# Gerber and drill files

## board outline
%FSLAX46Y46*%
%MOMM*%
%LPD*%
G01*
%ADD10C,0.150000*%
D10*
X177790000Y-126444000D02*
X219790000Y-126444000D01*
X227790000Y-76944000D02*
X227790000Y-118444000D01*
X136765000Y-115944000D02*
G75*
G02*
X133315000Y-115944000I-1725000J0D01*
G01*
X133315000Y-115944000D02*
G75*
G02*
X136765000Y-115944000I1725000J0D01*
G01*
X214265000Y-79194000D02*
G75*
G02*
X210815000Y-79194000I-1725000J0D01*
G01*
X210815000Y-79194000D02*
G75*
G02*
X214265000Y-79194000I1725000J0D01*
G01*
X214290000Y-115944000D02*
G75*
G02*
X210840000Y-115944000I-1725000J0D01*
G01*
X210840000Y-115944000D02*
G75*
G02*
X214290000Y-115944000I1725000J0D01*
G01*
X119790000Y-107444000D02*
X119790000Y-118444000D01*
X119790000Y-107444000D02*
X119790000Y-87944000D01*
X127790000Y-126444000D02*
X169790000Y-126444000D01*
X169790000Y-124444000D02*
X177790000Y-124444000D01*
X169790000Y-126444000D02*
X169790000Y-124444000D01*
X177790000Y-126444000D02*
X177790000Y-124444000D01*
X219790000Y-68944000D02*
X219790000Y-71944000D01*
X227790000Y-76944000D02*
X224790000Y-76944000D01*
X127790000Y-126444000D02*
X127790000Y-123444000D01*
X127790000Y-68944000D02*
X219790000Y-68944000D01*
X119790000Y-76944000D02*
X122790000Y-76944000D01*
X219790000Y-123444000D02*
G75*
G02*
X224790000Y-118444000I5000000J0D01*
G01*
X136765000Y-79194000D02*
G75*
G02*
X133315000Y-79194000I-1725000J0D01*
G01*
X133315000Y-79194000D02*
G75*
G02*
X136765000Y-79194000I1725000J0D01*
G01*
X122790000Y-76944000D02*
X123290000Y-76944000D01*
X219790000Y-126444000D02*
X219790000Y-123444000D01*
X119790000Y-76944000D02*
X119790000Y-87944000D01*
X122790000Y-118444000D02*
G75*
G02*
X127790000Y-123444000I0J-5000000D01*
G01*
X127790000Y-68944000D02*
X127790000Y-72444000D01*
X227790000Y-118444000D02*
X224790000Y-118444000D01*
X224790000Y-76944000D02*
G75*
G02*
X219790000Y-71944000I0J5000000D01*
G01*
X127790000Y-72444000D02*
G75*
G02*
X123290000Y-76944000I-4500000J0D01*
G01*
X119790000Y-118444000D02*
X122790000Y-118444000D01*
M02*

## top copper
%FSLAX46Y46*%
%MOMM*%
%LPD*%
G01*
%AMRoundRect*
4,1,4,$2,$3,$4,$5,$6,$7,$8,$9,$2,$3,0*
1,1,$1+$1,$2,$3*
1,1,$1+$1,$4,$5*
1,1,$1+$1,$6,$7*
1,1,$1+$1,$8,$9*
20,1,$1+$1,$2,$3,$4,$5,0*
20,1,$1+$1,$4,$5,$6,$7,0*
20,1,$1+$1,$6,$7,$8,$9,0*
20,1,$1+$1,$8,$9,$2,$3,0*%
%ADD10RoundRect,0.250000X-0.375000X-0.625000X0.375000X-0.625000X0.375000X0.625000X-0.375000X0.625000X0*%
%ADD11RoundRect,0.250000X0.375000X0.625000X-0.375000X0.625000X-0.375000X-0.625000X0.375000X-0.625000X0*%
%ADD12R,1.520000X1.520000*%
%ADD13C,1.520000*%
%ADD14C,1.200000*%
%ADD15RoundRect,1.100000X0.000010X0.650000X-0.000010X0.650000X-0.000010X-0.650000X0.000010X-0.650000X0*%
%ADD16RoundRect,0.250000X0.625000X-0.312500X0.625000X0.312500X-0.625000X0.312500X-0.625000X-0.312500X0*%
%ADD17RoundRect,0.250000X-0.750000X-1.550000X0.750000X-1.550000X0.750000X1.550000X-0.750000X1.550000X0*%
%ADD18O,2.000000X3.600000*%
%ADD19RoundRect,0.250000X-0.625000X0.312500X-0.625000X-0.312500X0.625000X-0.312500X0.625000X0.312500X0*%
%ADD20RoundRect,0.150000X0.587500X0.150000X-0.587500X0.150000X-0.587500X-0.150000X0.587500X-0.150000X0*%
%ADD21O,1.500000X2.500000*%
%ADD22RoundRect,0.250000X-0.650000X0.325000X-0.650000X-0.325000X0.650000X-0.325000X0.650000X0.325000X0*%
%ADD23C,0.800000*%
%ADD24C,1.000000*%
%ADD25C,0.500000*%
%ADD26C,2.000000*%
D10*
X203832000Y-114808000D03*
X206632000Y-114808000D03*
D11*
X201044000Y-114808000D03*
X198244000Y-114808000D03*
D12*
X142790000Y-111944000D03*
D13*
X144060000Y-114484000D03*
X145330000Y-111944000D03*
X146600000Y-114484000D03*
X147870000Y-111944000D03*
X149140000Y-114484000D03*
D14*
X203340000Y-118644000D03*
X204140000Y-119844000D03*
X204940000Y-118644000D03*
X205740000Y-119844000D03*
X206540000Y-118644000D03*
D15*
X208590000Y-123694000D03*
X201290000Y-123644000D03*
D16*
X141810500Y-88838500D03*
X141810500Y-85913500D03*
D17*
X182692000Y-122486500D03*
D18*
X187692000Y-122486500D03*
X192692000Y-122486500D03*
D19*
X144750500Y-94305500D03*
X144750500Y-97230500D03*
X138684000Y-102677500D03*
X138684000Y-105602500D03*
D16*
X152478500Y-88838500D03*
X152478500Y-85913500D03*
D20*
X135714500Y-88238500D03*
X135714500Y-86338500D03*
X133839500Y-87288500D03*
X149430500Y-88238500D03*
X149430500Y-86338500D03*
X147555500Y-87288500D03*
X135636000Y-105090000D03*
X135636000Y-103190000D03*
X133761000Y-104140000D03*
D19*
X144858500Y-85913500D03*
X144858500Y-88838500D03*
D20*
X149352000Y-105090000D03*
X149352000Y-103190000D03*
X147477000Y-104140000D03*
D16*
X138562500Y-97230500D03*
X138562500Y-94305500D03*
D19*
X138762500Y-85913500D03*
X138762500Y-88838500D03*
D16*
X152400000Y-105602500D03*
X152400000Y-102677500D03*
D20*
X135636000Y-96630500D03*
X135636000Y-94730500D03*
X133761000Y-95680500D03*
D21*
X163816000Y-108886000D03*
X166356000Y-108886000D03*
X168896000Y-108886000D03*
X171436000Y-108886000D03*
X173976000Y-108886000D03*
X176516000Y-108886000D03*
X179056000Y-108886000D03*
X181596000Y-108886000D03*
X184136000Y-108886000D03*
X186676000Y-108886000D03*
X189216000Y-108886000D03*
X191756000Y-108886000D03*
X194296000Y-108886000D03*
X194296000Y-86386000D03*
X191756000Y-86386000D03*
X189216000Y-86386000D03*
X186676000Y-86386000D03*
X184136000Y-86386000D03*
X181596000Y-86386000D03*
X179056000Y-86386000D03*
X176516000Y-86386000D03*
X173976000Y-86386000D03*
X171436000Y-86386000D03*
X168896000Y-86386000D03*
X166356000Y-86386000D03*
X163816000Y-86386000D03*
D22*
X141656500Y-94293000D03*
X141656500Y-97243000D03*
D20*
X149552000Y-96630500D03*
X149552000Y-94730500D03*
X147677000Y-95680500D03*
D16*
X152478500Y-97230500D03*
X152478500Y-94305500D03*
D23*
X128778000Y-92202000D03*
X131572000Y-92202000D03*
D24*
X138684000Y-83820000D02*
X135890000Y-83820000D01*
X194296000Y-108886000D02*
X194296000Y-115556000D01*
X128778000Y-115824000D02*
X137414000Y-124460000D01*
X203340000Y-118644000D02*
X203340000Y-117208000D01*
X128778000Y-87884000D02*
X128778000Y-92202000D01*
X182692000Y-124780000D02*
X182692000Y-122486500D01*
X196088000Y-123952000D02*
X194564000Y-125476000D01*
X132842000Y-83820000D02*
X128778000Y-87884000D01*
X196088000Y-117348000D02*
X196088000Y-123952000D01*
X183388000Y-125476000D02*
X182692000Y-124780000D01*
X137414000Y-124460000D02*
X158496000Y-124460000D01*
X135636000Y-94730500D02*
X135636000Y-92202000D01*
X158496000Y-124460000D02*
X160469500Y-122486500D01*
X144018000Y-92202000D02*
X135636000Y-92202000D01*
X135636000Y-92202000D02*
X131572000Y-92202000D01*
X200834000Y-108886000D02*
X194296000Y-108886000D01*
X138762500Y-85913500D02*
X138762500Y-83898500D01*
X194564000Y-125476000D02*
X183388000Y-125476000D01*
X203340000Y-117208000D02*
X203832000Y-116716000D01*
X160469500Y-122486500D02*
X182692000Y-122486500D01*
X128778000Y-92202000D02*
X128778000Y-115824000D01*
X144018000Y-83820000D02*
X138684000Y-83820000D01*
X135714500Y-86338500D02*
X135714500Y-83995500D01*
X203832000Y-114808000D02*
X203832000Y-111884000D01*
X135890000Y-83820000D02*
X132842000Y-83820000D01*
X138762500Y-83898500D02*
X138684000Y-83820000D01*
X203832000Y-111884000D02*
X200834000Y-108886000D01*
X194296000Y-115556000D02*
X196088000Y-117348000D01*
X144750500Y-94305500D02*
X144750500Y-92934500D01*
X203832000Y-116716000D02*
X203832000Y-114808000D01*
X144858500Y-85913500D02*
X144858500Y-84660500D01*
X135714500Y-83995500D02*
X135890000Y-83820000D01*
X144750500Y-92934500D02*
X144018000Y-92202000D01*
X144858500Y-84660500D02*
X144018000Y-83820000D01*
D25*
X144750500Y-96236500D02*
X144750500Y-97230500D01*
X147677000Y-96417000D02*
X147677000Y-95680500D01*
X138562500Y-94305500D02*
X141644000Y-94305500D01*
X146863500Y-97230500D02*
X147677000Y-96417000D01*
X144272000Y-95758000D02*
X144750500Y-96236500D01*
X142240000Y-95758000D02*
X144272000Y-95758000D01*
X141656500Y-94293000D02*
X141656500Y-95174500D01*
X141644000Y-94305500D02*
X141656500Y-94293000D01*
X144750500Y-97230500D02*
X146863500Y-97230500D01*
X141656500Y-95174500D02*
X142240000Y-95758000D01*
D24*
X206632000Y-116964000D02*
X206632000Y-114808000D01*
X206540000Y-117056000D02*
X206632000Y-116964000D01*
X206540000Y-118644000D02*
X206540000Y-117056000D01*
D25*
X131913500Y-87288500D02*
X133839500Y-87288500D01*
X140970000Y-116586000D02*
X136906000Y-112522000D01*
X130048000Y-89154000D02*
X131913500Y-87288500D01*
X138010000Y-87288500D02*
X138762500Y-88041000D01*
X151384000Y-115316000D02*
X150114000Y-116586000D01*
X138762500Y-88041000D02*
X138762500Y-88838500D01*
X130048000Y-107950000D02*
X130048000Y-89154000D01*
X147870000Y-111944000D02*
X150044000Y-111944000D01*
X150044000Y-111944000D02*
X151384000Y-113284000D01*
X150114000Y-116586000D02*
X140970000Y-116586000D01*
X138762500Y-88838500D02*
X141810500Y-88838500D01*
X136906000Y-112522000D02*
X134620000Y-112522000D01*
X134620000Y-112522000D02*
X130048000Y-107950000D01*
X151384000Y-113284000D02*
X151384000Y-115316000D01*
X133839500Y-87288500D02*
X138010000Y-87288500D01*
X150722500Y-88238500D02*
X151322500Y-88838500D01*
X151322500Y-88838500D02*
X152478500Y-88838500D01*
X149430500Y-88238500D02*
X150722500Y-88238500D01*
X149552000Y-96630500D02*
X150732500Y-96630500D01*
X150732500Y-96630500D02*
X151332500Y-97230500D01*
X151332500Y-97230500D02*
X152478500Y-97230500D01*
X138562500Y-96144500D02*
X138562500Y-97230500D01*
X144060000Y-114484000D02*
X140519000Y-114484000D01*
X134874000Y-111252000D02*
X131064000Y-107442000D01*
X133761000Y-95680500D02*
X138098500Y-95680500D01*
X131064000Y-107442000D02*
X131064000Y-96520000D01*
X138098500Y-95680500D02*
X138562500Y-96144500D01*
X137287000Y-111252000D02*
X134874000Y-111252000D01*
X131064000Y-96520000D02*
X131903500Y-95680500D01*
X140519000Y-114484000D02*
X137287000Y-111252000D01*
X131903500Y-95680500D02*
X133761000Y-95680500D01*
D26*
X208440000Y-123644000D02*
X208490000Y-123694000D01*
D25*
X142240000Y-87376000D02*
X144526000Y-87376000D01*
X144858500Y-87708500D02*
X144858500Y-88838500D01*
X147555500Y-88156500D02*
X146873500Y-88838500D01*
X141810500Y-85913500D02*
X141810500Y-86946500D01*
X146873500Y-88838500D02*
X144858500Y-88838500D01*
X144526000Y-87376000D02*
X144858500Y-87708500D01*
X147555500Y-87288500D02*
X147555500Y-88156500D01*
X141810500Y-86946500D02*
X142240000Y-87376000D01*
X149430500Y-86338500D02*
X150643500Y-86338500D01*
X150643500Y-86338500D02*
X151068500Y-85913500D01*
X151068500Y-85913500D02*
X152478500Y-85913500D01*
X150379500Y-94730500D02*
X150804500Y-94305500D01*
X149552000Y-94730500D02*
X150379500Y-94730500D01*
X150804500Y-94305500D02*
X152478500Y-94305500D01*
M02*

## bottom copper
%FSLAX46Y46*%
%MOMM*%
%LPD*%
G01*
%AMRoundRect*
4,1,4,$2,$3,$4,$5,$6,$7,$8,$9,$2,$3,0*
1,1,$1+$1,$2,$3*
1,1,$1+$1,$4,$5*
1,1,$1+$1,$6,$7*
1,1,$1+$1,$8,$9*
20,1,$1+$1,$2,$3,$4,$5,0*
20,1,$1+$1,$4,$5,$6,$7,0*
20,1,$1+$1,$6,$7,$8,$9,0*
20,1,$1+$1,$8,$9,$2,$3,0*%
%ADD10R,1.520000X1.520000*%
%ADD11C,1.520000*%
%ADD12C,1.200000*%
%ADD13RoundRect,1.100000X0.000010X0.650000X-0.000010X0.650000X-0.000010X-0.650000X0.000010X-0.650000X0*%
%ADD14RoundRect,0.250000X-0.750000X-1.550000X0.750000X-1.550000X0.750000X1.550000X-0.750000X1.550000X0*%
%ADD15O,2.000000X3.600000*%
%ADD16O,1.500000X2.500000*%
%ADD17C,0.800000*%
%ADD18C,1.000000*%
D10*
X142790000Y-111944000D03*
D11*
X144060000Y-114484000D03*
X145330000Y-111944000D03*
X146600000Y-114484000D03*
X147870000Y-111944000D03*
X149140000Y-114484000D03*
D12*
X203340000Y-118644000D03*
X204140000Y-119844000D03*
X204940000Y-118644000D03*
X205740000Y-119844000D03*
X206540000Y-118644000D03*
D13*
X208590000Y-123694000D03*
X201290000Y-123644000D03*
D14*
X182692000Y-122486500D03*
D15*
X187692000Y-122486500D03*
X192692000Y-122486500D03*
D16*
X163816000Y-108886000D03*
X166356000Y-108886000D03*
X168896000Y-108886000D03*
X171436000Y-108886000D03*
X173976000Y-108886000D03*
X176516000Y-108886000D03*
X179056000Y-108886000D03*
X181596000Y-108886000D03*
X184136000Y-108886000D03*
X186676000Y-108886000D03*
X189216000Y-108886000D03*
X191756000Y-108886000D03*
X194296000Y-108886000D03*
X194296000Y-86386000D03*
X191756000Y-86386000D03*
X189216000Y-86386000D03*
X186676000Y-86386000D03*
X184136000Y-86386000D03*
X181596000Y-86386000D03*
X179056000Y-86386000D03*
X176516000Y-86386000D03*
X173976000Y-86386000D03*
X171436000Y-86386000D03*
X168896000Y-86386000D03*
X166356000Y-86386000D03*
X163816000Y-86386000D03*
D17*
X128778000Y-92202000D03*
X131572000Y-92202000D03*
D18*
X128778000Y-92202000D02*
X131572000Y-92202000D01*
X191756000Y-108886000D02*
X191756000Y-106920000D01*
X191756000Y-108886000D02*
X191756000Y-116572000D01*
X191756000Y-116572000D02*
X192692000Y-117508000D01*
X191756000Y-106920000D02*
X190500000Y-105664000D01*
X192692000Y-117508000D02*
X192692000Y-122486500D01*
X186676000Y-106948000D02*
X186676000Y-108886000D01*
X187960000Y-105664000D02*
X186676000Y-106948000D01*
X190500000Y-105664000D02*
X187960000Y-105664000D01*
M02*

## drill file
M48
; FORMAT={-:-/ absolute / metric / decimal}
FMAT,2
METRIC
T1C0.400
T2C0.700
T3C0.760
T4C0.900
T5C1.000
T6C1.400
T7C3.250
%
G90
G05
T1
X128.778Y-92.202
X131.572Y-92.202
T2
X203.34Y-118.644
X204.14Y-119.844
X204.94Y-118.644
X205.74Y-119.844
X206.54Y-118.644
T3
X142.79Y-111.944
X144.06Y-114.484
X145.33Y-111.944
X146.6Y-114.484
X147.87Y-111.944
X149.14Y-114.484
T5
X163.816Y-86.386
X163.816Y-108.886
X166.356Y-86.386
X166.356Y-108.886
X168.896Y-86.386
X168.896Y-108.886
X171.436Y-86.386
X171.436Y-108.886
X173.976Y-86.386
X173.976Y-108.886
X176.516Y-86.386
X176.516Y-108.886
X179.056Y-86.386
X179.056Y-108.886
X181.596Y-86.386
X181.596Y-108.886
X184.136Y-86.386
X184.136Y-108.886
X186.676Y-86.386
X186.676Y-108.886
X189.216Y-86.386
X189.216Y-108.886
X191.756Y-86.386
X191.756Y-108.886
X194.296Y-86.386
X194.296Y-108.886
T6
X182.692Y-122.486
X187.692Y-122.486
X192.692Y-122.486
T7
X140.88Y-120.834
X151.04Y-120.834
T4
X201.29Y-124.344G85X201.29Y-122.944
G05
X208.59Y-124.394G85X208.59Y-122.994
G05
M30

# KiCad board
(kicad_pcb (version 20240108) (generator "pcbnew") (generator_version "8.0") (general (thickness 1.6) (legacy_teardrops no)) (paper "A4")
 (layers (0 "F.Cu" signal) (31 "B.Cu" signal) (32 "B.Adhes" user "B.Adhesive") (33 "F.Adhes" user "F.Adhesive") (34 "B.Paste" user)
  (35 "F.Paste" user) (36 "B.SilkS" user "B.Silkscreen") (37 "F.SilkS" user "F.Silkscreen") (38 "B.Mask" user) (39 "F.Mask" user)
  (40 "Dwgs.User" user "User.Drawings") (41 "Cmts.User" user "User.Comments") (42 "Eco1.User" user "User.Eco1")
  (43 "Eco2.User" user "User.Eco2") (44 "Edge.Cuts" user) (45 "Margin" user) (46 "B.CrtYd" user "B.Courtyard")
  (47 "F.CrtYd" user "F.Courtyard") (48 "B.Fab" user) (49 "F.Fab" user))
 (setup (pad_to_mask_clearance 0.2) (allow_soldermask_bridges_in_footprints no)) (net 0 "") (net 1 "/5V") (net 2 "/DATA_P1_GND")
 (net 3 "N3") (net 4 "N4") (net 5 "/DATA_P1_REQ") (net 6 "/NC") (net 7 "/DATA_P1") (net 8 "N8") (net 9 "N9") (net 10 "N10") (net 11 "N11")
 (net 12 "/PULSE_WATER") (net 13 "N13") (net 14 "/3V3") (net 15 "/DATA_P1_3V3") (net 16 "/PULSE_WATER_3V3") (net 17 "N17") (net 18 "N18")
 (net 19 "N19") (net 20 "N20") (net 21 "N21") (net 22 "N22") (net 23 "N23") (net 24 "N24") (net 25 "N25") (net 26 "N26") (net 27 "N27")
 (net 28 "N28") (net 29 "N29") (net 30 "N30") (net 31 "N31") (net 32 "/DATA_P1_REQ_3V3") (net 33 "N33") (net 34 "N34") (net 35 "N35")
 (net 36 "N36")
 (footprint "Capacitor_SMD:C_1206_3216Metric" (layer "F.Cu") (at 205.232 114.808)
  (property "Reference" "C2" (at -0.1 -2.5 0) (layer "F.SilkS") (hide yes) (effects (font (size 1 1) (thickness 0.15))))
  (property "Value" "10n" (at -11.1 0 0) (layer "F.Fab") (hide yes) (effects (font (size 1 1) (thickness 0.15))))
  (pad "1" smd roundrect (at -1.4 0) (size 1.25 1.75) (layers "F.Cu" "F.Paste" "F.Mask") (roundrect_rratio 0.2) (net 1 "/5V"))
  (pad "2" smd roundrect (at 1.4 0) (size 1.25 1.75) (layers "F.Cu" "F.Paste" "F.Mask") (roundrect_rratio 0.2) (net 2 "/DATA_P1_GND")))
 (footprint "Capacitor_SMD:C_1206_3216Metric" (layer "F.Cu") (at 199.644 114.808 180)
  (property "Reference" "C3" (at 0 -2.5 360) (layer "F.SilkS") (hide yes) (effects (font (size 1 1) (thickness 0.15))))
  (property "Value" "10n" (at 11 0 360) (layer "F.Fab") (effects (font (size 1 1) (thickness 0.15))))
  (pad "1" smd roundrect (at -1.4 0 180) (size 1.25 1.75) (layers "F.Cu" "F.Paste" "F.Mask") (roundrect_rratio 0.2) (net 2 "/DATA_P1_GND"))
  (pad "2" smd roundrect (at 1.4 0 180) (size 1.25 1.75) (layers "F.Cu" "F.Paste" "F.Mask") (roundrect_rratio 0.2) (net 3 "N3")))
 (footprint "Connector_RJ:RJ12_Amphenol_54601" (layer "F.Cu") (at 142.79 111.944)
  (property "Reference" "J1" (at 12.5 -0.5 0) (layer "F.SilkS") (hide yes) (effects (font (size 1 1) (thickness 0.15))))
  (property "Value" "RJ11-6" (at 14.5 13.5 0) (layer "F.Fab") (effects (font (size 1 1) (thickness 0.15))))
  (pad "" np_thru_hole circle (at -1.91 8.89) (size 3.25 3.25) (drill 3.25) (layers "*.Cu" "*.Mask"))
  (pad "" np_thru_hole circle (at 8.25 8.89) (size 3.25 3.25) (drill 3.25) (layers "*.Cu" "*.Mask"))
  (pad "1" thru_hole rect (at 0 0) (size 1.52 1.52) (drill 0.76) (layers "*.Cu" "*.Mask") (remove_unused_layers no) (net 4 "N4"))
  (pad "2" thru_hole circle (at 1.27 2.54) (size 1.52 1.52) (drill 0.76) (layers "*.Cu" "*.Mask") (remove_unused_layers no)
   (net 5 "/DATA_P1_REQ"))
  (pad "3" thru_hole circle (at 2.54 0) (size 1.52 1.52) (drill 0.76) (layers "*.Cu" "*.Mask") (remove_unused_layers no)
   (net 2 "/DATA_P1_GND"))
  (pad "4" thru_hole circle (at 3.81 2.54) (size 1.52 1.52) (drill 0.76) (layers "*.Cu" "*.Mask") (remove_unused_layers no) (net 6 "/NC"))
  (pad "5" thru_hole circle (at 5.08 0) (size 1.52 1.52) (drill 0.76) (layers "*.Cu" "*.Mask") (remove_unused_layers no) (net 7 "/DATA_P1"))
  (pad "6" thru_hole circle (at 6.35 2.54) (size 1.52 1.52) (drill 0.76) (layers "*.Cu" "*.Mask") (remove_unused_layers no)
   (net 2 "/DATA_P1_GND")))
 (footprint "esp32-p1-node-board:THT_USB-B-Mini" (layer "F.Cu") (at 208.79 127.444 90)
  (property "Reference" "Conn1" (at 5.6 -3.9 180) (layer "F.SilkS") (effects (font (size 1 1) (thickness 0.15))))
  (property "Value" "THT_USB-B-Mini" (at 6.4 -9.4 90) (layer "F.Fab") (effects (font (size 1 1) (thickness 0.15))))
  (pad "1" thru_hole circle (at 8.8 -5.45 180) (size 1.2 1.2) (drill 0.7) (layers "*.Cu" "*.Mask") (remove_unused_layers no) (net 1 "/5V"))
  (pad "2" thru_hole circle (at 7.6 -4.65 180) (size 1.2 1.2) (drill 0.7) (layers "*.Cu" "*.Mask") (remove_unused_layers no) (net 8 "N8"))
  (pad "3" thru_hole circle (at 8.8 -3.85 180) (size 1.2 1.2) (drill 0.7) (layers "*.Cu" "*.Mask") (remove_unused_layers no) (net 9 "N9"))
  (pad "4" thru_hole circle (at 7.6 -3.05 180) (size 1.2 1.2) (drill 0.7) (layers "*.Cu" "*.Mask") (remove_unused_layers no) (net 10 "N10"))
  (pad "5" thru_hole circle (at 8.8 -2.25 180) (size 1.2 1.2) (drill 0.7) (layers "*.Cu" "*.Mask") (remove_unused_layers no)
   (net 2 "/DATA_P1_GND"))
  (pad "6" thru_hole roundrect (at 3.75 -0.2 180) (size 2.2 3.5) (drill oval 0.9 2.3) (layers "*.Cu" "*.Mask") (remove_unused_layers no)
   (roundrect_rratio 0.5) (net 3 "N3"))
  (pad "7" thru_hole roundrect (at 3.8 -7.5 180) (size 2.2 3.5) (drill oval 0.9 2.3) (layers "*.Cu" "*.Mask") (remove_unused_layers no)
   (roundrect_rratio 0.5) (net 3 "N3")))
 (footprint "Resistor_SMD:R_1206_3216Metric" (layer "F.Cu") (at 141.8105 87.376 90)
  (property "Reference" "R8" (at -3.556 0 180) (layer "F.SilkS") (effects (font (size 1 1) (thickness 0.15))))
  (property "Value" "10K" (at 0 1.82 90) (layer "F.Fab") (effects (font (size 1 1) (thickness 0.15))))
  (pad "1" smd roundrect (at -1.4625 0 90) (size 1.125 1.75) (layers "F.Cu" "F.Paste" "F.Mask") (roundrect_rratio 0.222222)
   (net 7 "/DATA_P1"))
  (pad "2" smd roundrect (at 1.4625 0 90) (size 1.125 1.75) (layers "F.Cu" "F.Paste" "F.Mask") (roundrect_rratio 0.222222) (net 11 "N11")))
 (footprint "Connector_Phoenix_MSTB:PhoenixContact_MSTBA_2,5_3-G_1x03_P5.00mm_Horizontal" (layer "F.Cu") (at 182.692 122.4865)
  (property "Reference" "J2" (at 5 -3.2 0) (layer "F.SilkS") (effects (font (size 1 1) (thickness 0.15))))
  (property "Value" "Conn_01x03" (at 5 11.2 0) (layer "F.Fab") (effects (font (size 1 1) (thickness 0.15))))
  (pad "1" thru_hole roundrect (at 0 0) (size 2 3.6) (drill 1.4) (layers "*.Cu" "*.Mask") (remove_unused_layers no) (roundrect_rratio 0.125)
   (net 1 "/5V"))
  (pad "2" thru_hole oval (at 5 0) (size 2 3.6) (drill 1.4) (layers "*.Cu" "*.Mask") (remove_unused_layers no) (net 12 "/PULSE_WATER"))
  (pad "3" thru_hole oval (at 10 0) (size 2 3.6) (drill 1.4) (layers "*.Cu" "*.Mask") (remove_unused_layers no) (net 2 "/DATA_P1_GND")))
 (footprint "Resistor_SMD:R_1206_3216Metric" (layer "F.Cu") (at 144.7505 95.768 -90)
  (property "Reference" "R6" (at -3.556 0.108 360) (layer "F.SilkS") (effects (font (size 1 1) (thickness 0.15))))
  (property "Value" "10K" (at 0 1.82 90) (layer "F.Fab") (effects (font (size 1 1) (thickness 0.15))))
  (pad "1" smd roundrect (at -1.4625 0 270) (size 1.125 1.75) (layers "F.Cu" "F.Paste" "F.Mask") (roundrect_rratio 0.222222) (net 1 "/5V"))
  (pad "2" smd roundrect (at 1.4625 0 270) (size 1.125 1.75) (layers "F.Cu" "F.Paste" "F.Mask") (roundrect_rratio 0.222222) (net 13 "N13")))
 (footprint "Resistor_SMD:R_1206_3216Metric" (layer "F.Cu") (at 138.684 104.14 -90)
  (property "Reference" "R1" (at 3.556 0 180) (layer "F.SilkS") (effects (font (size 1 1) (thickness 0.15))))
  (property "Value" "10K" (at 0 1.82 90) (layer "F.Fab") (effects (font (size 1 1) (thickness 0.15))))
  (pad "1" smd roundrect (at -1.4625 0 270) (size 1.125 1.75) (layers "F.Cu" "F.Paste" "F.Mask") (roundrect_rratio 0.222222) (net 1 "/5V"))
  (pad "2" smd roundrect (at 1.4625 0 270) (size 1.125 1.75) (layers "F.Cu" "F.Paste" "F.Mask") (roundrect_rratio 0.222222)
   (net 12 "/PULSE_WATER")))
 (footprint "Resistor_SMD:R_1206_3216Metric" (layer "F.Cu") (at 152.4785 87.376 90)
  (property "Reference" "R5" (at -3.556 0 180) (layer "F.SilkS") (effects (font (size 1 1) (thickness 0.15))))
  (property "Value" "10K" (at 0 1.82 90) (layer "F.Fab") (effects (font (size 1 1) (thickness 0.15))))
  (pad "1" smd roundrect (at -1.4625 0 90) (size 1.125 1.75) (layers "F.Cu" "F.Paste" "F.Mask") (roundrect_rratio 0.222222) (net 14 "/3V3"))
  (pad "2" smd roundrect (at 1.4625 0 90) (size 1.125 1.75) (layers "F.Cu" "F.Paste" "F.Mask") (roundrect_rratio 0.222222)
   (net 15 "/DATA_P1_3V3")))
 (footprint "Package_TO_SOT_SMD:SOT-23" (layer "F.Cu") (at 134.777 87.2885 180)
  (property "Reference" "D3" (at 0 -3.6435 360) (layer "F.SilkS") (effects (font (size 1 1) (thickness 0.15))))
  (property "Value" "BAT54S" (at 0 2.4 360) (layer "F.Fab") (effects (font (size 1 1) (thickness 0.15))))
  (pad "1" smd roundrect (at -0.9375 -0.95 180) (size 1.475 0.6) (layers "F.Cu" "F.Paste" "F.Mask") (roundrect_rratio 0.25)
   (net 2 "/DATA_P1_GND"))
  (pad "2" smd roundrect (at -0.9375 0.95 180) (size 1.475 0.6) (layers "F.Cu" "F.Paste" "F.Mask") (roundrect_rratio 0.25) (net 1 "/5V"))
  (pad "3" smd roundrect (at 0.9375 0 180) (size 1.475 0.6) (layers "F.Cu" "F.Paste" "F.Mask") (roundrect_rratio 0.25) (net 7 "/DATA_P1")))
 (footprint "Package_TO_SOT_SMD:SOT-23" (layer "F.Cu") (at 148.493 87.2885 180)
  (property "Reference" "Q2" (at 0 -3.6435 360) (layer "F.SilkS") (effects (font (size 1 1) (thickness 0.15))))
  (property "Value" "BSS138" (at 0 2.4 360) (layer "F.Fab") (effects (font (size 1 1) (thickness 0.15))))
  (pad "1" smd roundrect (at -0.9375 -0.95 180) (size 1.475 0.6) (layers "F.Cu" "F.Paste" "F.Mask") (roundrect_rratio 0.25) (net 14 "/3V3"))
  (pad "2" smd roundrect (at -0.9375 0.95 180) (size 1.475 0.6) (layers "F.Cu" "F.Paste" "F.Mask") (roundrect_rratio 0.25)
   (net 15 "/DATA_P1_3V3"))
  (pad "3" smd roundrect (at 0.9375 0 180) (size 1.475 0.6) (layers "F.Cu" "F.Paste" "F.Mask") (roundrect_rratio 0.25) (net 11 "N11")))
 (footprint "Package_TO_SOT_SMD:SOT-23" (layer "F.Cu") (at 134.6985 104.14 180)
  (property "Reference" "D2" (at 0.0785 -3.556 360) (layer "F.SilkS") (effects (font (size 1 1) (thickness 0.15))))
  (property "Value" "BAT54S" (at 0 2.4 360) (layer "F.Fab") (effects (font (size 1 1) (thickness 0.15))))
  (pad "1" smd roundrect (at -0.9375 -0.95 180) (size 1.475 0.6) (layers "F.Cu" "F.Paste" "F.Mask") (roundrect_rratio 0.25)
   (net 2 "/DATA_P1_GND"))
  (pad "2" smd roundrect (at -0.9375 0.95 180) (size 1.475 0.6) (layers "F.Cu" "F.Paste" "F.Mask") (roundrect_rratio 0.25) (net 1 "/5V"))
  (pad "3" smd roundrect (at 0.9375 0 180) (size 1.475 0.6) (layers "F.Cu" "F.Paste" "F.Mask") (roundrect_rratio 0.25)
   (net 12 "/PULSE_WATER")))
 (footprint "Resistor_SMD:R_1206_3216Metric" (layer "F.Cu") (at 144.8585 87.376 -90)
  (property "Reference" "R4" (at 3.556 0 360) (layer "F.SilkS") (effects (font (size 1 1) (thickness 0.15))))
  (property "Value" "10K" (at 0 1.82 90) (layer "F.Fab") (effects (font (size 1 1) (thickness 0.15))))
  (pad "1" smd roundrect (at -1.4625 0 270) (size 1.125 1.75) (layers "F.Cu" "F.Paste" "F.Mask") (roundrect_rratio 0.222222) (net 1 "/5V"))
  (pad "2" smd roundrect (at 1.4625 0 270) (size 1.125 1.75) (layers "F.Cu" "F.Paste" "F.Mask") (roundrect_rratio 0.222222) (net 11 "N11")))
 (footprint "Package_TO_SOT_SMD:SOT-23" (layer "F.Cu") (at 148.4145 104.14 180)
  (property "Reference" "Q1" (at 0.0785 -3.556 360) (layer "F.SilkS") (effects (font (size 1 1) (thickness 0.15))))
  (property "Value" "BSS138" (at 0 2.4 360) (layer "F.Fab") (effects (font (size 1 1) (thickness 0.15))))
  (pad "1" smd roundrect (at -0.9375 -0.95 180) (size 1.475 0.6) (layers "F.Cu" "F.Paste" "F.Mask") (roundrect_rratio 0.25) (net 14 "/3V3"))
  (pad "2" smd roundrect (at -0.9375 0.95 180) (size 1.475 0.6) (layers "F.Cu" "F.Paste" "F.Mask") (roundrect_rratio 0.25)
   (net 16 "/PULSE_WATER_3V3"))
  (pad "3" smd roundrect (at 0.9375 0 180) (size 1.475 0.6) (layers "F.Cu" "F.Paste" "F.Mask") (roundrect_rratio 0.25)
   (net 12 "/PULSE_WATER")))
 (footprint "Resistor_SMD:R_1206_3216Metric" (layer "F.Cu") (at 138.5625 95.768 90)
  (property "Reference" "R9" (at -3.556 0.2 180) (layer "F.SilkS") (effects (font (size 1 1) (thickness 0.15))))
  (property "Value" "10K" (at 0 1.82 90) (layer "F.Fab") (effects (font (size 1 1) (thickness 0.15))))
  (pad "1" smd roundrect (at -1.4625 0 90) (size 1.125 1.75) (layers "F.Cu" "F.Paste" "F.Mask") (roundrect_rratio 0.222222)
   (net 5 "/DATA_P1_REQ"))
  (pad "2" smd roundrect (at 1.4625 0 90) (size 1.125 1.75) (layers "F.Cu" "F.Paste" "F.Mask") (roundrect_rratio 0.222222) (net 13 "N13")))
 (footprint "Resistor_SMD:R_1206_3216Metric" (layer "F.Cu") (at 138.7625 87.376 -90)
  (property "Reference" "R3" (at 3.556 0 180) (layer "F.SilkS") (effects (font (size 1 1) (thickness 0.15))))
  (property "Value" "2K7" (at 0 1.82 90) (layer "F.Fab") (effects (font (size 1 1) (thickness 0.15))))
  (pad "1" smd roundrect (at -1.4625 0 270) (size 1.125 1.75) (layers "F.Cu" "F.Paste" "F.Mask") (roundrect_rratio 0.222222) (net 1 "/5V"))
  (pad "2" smd roundrect (at 1.4625 0 270) (size 1.125 1.75) (layers "F.Cu" "F.Paste" "F.Mask") (roundrect_rratio 0.222222)
   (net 7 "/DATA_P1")))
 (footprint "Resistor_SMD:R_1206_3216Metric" (layer "F.Cu") (at 152.4 104.14 90)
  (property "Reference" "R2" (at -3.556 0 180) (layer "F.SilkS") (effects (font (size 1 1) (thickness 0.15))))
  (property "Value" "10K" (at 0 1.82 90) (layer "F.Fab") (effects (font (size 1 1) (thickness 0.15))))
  (pad "1" smd roundrect (at -1.4625 0 90) (size 1.125 1.75) (layers "F.Cu" "F.Paste" "F.Mask") (roundrect_rratio 0.222222) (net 14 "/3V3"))
  (pad "2" smd roundrect (at 1.4625 0 90) (size 1.125 1.75) (layers "F.Cu" "F.Paste" "F.Mask") (roundrect_rratio 0.222222)
   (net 16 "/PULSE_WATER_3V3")))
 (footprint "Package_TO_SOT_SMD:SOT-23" (layer "F.Cu") (at 134.6985 95.6805 180)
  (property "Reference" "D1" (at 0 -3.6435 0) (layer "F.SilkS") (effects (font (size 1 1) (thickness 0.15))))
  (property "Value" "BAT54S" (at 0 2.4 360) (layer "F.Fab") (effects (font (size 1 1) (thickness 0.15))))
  (pad "1" smd roundrect (at -0.9375 -0.95 180) (size 1.475 0.6) (layers "F.Cu" "F.Paste" "F.Mask") (roundrect_rratio 0.25)
   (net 2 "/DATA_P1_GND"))
  (pad "2" smd roundrect (at -0.9375 0.95 180) (size 1.475 0.6) (layers "F.Cu" "F.Paste" "F.Mask") (roundrect_rratio 0.25) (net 1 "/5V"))
  (pad "3" smd roundrect (at 0.9375 0 180) (size 1.475 0.6) (layers "F.Cu" "F.Paste" "F.Mask") (roundrect_rratio 0.25)
   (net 5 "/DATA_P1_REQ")))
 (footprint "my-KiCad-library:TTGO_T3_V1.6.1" (layer "F.Cu") (at 179.056 97.636)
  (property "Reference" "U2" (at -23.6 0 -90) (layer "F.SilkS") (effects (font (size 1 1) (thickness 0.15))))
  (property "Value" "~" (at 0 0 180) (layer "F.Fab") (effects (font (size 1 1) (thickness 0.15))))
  (pad "1" thru_hole oval (at -15.24 11.25) (size 1.5 2.5) (drill 1) (layers "*.Cu" "*.Mask") (remove_unused_layers no) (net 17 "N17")
   (thermal_bridge_angle 45))
  (pad "2" thru_hole oval (at -12.7 11.25) (size 1.5 2.5) (drill 1) (layers "*.Cu" "*.Mask") (remove_unused_layers no) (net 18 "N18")
   (thermal_bridge_angle 45))
  (pad "3" thru_hole oval (at -10.16 11.25) (size 1.5 2.5) (drill 1) (layers "*.Cu" "*.Mask") (remove_unused_layers no) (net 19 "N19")
   (thermal_bridge_angle 45))
  (pad "4" thru_hole oval (at -7.62 11.25) (size 1.5 2.5) (drill 1) (layers "*.Cu" "*.Mask") (remove_unused_layers no) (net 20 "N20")
   (thermal_bridge_angle 45))
  (pad "5" thru_hole oval (at -5.08 11.25) (size 1.5 2.5) (drill 1) (layers "*.Cu" "*.Mask") (remove_unused_layers no) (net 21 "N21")
   (thermal_bridge_angle 45))
  (pad "6" thru_hole oval (at -2.54 11.25) (size 1.5 2.5) (drill 1) (layers "*.Cu" "*.Mask") (remove_unused_layers no) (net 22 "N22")
   (thermal_bridge_angle 45))
  (pad "7" thru_hole oval (at 0 11.25) (size 1.5 2.5) (drill 1) (layers "*.Cu" "*.Mask") (remove_unused_layers no) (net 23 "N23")
   (thermal_bridge_angle 45))
  (pad "8" thru_hole oval (at 2.54 11.25) (size 1.5 2.5) (drill 1) (layers "*.Cu" "*.Mask") (remove_unused_layers no) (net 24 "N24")
   (thermal_bridge_angle 45))
  (pad "9" thru_hole oval (at 5.08 11.25) (size 1.5 2.5) (drill 1) (layers "*.Cu" "*.Mask") (remove_unused_layers no) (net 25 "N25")
   (thermal_bridge_angle 45))
  (pad "10" thru_hole oval (at 7.62 11.25) (size 1.5 2.5) (drill 1) (layers "*.Cu" "*.Mask") (remove_unused_layers no)
   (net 2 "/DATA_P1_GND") (thermal_bridge_angle 45))
  (pad "11" thru_hole oval (at 10.16 11.25) (size 1.5 2.5) (drill 1) (layers "*.Cu" "*.Mask") (remove_unused_layers no) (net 14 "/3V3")
   (thermal_bridge_angle 45))
  (pad "12" thru_hole oval (at 12.7 11.25) (size 1.5 2.5) (drill 1) (layers "*.Cu" "*.Mask") (remove_unused_layers no)
   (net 2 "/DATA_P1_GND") (thermal_bridge_angle 45))
  (pad "13" thru_hole oval (at 15.24 11.25) (size 1.5 2.5) (drill 1) (layers "*.Cu" "*.Mask") (remove_unused_layers no) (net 1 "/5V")
   (thermal_bridge_angle 45))
  (pad "14" thru_hole oval (at 15.24 -11.25) (size 1.5 2.5) (drill 1) (layers "*.Cu" "*.Mask") (remove_unused_layers no) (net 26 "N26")
   (thermal_bridge_angle 45))
  (pad "15" thru_hole oval (at 12.7 -11.25) (size 1.5 2.5) (drill 1) (layers "*.Cu" "*.Mask") (remove_unused_layers no)
   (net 16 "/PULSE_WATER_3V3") (thermal_bridge_angle 45))
  (pad "16" thru_hole oval (at 10.16 -11.25) (size 1.5 2.5) (drill 1) (layers "*.Cu" "*.Mask") (remove_unused_layers no) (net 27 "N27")
   (thermal_bridge_angle 45))
  (pad "17" thru_hole oval (at 7.62 -11.25) (size 1.5 2.5) (drill 1) (layers "*.Cu" "*.Mask") (remove_unused_layers no) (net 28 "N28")
   (thermal_bridge_angle 45))
  (pad "18" thru_hole oval (at 5.08 -11.25) (size 1.5 2.5) (drill 1) (layers "*.Cu" "*.Mask") (remove_unused_layers no) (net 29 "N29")
   (thermal_bridge_angle 45))
  (pad "19" thru_hole oval (at 2.54 -11.25) (size 1.5 2.5) (drill 1) (layers "*.Cu" "*.Mask") (remove_unused_layers no) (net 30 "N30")
   (thermal_bridge_angle 45))
  (pad "20" thru_hole oval (at 0 -11.25) (size 1.5 2.5) (drill 1) (layers "*.Cu" "*.Mask") (remove_unused_layers no) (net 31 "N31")
   (thermal_bridge_angle 45))
  (pad "21" thru_hole oval (at -2.54 -11.25) (size 1.5 2.5) (drill 1) (layers "*.Cu" "*.Mask") (remove_unused_layers no)
   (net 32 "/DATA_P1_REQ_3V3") (thermal_bridge_angle 45))
  (pad "22" thru_hole oval (at -5.08 -11.25) (size 1.5 2.5) (drill 1) (layers "*.Cu" "*.Mask") (remove_unused_layers no) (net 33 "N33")
   (thermal_bridge_angle 45))
  (pad "23" thru_hole oval (at -7.62 -11.25) (size 1.5 2.5) (drill 1) (layers "*.Cu" "*.Mask") (remove_unused_layers no)
   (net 15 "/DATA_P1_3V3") (thermal_bridge_angle 45))
  (pad "24" thru_hole oval (at -10.16 -11.25) (size 1.5 2.5) (drill 1) (layers "*.Cu" "*.Mask") (remove_unused_layers no) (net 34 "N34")
   (thermal_bridge_angle 45))
  (pad "25" thru_hole oval (at -12.7 -11.25) (size 1.5 2.5) (drill 1) (layers "*.Cu" "*.Mask") (remove_unused_layers no) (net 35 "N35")
   (thermal_bridge_angle 45))
  (pad "26" thru_hole oval (at -15.24 -11.25) (size 1.5 2.5) (drill 1) (layers "*.Cu" "*.Mask") (remove_unused_layers no) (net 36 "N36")
   (thermal_bridge_angle 45)))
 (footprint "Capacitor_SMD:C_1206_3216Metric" (layer "F.Cu") (at 141.6565 95.768 -90)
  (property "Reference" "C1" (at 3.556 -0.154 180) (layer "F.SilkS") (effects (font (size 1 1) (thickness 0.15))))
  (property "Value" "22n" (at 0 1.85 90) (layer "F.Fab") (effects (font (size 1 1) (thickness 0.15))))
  (pad "1" smd roundrect (at -1.475 0 270) (size 1.15 1.8) (layers "F.Cu" "F.Paste" "F.Mask") (roundrect_rratio 0.217391) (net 13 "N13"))
  (pad "2" smd roundrect (at 1.475 0 270) (size 1.15 1.8) (layers "F.Cu" "F.Paste" "F.Mask") (roundrect_rratio 0.217391)
   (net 2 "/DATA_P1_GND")))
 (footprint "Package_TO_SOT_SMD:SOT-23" (layer "F.Cu") (at 148.6145 95.6805 180)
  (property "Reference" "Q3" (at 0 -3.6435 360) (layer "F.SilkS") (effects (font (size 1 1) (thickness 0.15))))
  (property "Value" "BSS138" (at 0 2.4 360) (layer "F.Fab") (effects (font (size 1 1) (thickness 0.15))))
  (pad "1" smd roundrect (at -0.9375 -0.95 180) (size 1.475 0.6) (layers "F.Cu" "F.Paste" "F.Mask") (roundrect_rratio 0.25) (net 14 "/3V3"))
  (pad "2" smd roundrect (at -0.9375 0.95 180) (size 1.475 0.6) (layers "F.Cu" "F.Paste" "F.Mask") (roundrect_rratio 0.25)
   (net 32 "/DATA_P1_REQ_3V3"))
  (pad "3" smd roundrect (at 0.9375 0 180) (size 1.475 0.6) (layers "F.Cu" "F.Paste" "F.Mask") (roundrect_rratio 0.25) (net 13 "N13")))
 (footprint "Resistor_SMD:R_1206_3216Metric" (layer "F.Cu") (at 152.4785 95.768 90)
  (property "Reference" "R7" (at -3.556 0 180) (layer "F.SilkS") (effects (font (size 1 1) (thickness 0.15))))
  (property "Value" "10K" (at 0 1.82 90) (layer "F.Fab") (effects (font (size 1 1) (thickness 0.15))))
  (pad "1" smd roundrect (at -1.4625 0 90) (size 1.125 1.75) (layers "F.Cu" "F.Paste" "F.Mask") (roundrect_rratio 0.222222) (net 14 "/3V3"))
  (pad "2" smd roundrect (at 1.4625 0 90) (size 1.125 1.75) (layers "F.Cu" "F.Paste" "F.Mask") (roundrect_rratio 0.222222)
   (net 32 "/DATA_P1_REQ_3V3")))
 (gr_line (start 177.79 126.444) (end 219.79 126.444) (stroke (width 0.15) (type solid)) (layer "Edge.Cuts"))
 (gr_line (start 227.79 76.944) (end 227.79 118.444) (stroke (width 0.15) (type solid)) (layer "Edge.Cuts"))
 (gr_circle (center 135.04 115.944) (end 136.765 115.944) (stroke (width 0.15) (type solid)) (fill none) (layer "Edge.Cuts"))
 (gr_circle (center 212.54 79.194) (end 214.265 79.194) (stroke (width 0.15) (type solid)) (fill none) (layer "Edge.Cuts"))
 (gr_circle (center 212.565 115.944) (end 214.29 115.944) (stroke (width 0.15) (type solid)) (fill none) (layer "Edge.Cuts"))
 (gr_line (start 119.79 107.444) (end 119.79 118.444) (stroke (width 0.15) (type solid)) (layer "Edge.Cuts"))
 (gr_line (start 119.79 107.444) (end 119.79 87.944) (stroke (width 0.15) (type solid)) (layer "Edge.Cuts"))
 (gr_line (start 127.79 126.444) (end 169.79 126.444) (stroke (width 0.15) (type solid)) (layer "Edge.Cuts"))
 (gr_line (start 169.79 124.444) (end 177.79 124.444) (stroke (width 0.15) (type solid)) (layer "Edge.Cuts"))
 (gr_line (start 169.79 126.444) (end 169.79 124.444) (stroke (width 0.15) (type solid)) (layer "Edge.Cuts"))
 (gr_line (start 177.79 126.444) (end 177.79 124.444) (stroke (width 0.15) (type solid)) (layer "Edge.Cuts"))
 (gr_line (start 219.79 68.944) (end 219.79 71.944) (stroke (width 0.15) (type solid)) (layer "Edge.Cuts"))
 (gr_line (start 227.79 76.944) (end 224.79 76.944) (stroke (width 0.15) (type solid)) (layer "Edge.Cuts"))
 (gr_line (start 127.79 126.444) (end 127.79 123.444) (stroke (width 0.15) (type solid)) (layer "Edge.Cuts"))
 (gr_line (start 127.79 68.944) (end 219.79 68.944) (stroke (width 0.15) (type solid)) (layer "Edge.Cuts"))
 (gr_line (start 119.79 76.944) (end 122.79 76.944) (stroke (width 0.15) (type solid)) (layer "Edge.Cuts"))
 (gr_arc (start 219.79 123.444) (mid 221.254466 119.908466) (end 224.79 118.444) (stroke (width 0.15) (type solid)) (layer "Edge.Cuts"))
 (gr_circle (center 135.04 79.194) (end 136.765 79.194) (stroke (width 0.15) (type solid)) (fill none) (layer "Edge.Cuts"))
 (gr_line (start 122.79 76.944) (end 123.29 76.944) (stroke (width 0.15) (type solid)) (layer "Edge.Cuts"))
 (gr_line (start 219.79 126.444) (end 219.79 123.444) (stroke (width 0.15) (type solid)) (layer "Edge.Cuts"))
 (gr_line (start 119.79 76.944) (end 119.79 87.944) (stroke (width 0.15) (type solid)) (layer "Edge.Cuts"))
 (gr_arc (start 122.79 118.444) (mid 126.325534 119.908466) (end 127.79 123.444) (stroke (width 0.15) (type solid)) (layer "Edge.Cuts"))
 (gr_line (start 127.79 68.944) (end 127.79 72.444) (stroke (width 0.15) (type solid)) (layer "Edge.Cuts"))
 (gr_line (start 227.79 118.444) (end 224.79 118.444) (stroke (width 0.15) (type solid)) (layer "Edge.Cuts"))
 (gr_arc (start 224.79 76.944) (mid 221.254466 75.479534) (end 219.79 71.944) (stroke (width 0.15) (type solid)) (layer "Edge.Cuts"))
 (gr_arc (start 127.79 72.444) (mid 126.471981 75.625981) (end 123.29 76.944) (stroke (width 0.15) (type solid)) (layer "Edge.Cuts"))
 (gr_line (start 119.79 118.444) (end 122.79 118.444) (stroke (width 0.15) (type solid)) (layer "Edge.Cuts"))
 (segment (start 138.684 83.82) (end 135.89 83.82) (width 1) (layer "F.Cu") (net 1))
 (segment (start 194.296 108.886) (end 194.296 115.556) (width 1) (layer "F.Cu") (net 1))
 (segment (start 128.778 115.824) (end 137.414 124.46) (width 1) (layer "F.Cu") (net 1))
 (segment (start 203.34 118.644) (end 203.34 117.208) (width 1) (layer "F.Cu") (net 1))
 (segment (start 128.778 87.884) (end 128.778 92.202) (width 1) (layer "F.Cu") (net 1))
 (segment (start 182.692 124.78) (end 182.692 122.4865) (width 1) (layer "F.Cu") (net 1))
 (segment (start 196.088 123.952) (end 194.564 125.476) (width 1) (layer "F.Cu") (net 1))
 (segment (start 132.842 83.82) (end 128.778 87.884) (width 1) (layer "F.Cu") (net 1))
 (segment (start 196.088 117.348) (end 196.088 123.952) (width 1) (layer "F.Cu") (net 1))
 (segment (start 183.388 125.476) (end 182.692 124.78) (width 1) (layer "F.Cu") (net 1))
 (segment (start 137.414 124.46) (end 158.496 124.46) (width 1) (layer "F.Cu") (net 1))
 (segment (start 135.636 94.7305) (end 135.636 92.202) (width 1) (layer "F.Cu") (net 1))
 (segment (start 158.496 124.46) (end 160.4695 122.4865) (width 1) (layer "F.Cu") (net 1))
 (segment (start 144.018 92.202) (end 135.636 92.202) (width 1) (layer "F.Cu") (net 1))
 (segment (start 135.636 92.202) (end 131.572 92.202) (width 1) (layer "F.Cu") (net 1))
 (segment (start 200.834 108.886) (end 194.296 108.886) (width 1) (layer "F.Cu") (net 1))
 (segment (start 138.7625 85.9135) (end 138.7625 83.8985) (width 1) (layer "F.Cu") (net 1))
 (segment (start 194.564 125.476) (end 183.388 125.476) (width 1) (layer "F.Cu") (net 1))
 (segment (start 203.34 117.208) (end 203.832 116.716) (width 1) (layer "F.Cu") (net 1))
 (segment (start 160.4695 122.4865) (end 182.692 122.4865) (width 1) (layer "F.Cu") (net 1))
 (segment (start 128.778 92.202) (end 128.778 115.824) (width 1) (layer "F.Cu") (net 1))
 (segment (start 144.018 83.82) (end 138.684 83.82) (width 1) (layer "F.Cu") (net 1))
 (segment (start 135.7145 86.3385) (end 135.7145 83.9955) (width 1) (layer "F.Cu") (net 1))
 (segment (start 203.832 114.808) (end 203.832 111.884) (width 1) (layer "F.Cu") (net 1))
 (segment (start 135.89 83.82) (end 132.842 83.82) (width 1) (layer "F.Cu") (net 1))
 (segment (start 138.7625 83.8985) (end 138.684 83.82) (width 1) (layer "F.Cu") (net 1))
 (segment (start 203.832 111.884) (end 200.834 108.886) (width 1) (layer "F.Cu") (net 1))
 (segment (start 194.296 115.556) (end 196.088 117.348) (width 1) (layer "F.Cu") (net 1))
 (segment (start 144.7505 94.3055) (end 144.7505 92.9345) (width 1) (layer "F.Cu") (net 1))
 (segment (start 203.832 116.716) (end 203.832 114.808) (width 1) (layer "F.Cu") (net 1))
 (segment (start 144.8585 85.9135) (end 144.8585 84.6605) (width 1) (layer "F.Cu") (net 1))
 (segment (start 135.7145 83.9955) (end 135.89 83.82) (width 1) (layer "F.Cu") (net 1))
 (segment (start 144.7505 92.9345) (end 144.018 92.202) (width 1) (layer "F.Cu") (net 1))
 (segment (start 144.8585 84.6605) (end 144.018 83.82) (width 1) (layer "F.Cu") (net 1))
 (via (at 128.778 92.202) (size 0.8) (drill 0.4) (layers "F.Cu" "B.Cu") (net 1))
 (via (at 131.572 92.202) (size 0.8) (drill 0.4) (layers "F.Cu" "B.Cu") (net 1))
 (segment (start 128.778 92.202) (end 131.572 92.202) (width 1) (layer "B.Cu") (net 1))
 (segment (start 144.7505 96.2365) (end 144.7505 97.2305) (width 0.5) (layer "F.Cu") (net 13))
 (segment (start 147.677 96.417) (end 147.677 95.6805) (width 0.5) (layer "F.Cu") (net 13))
 (segment (start 138.5625 94.3055) (end 141.644 94.3055) (width 0.5) (layer "F.Cu") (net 13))
 (segment (start 146.8635 97.2305) (end 147.677 96.417) (width 0.5) (layer "F.Cu") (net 13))
 (segment (start 144.272 95.758) (end 144.7505 96.2365) (width 0.5) (layer "F.Cu") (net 13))
 (segment (start 142.24 95.758) (end 144.272 95.758) (width 0.5) (layer "F.Cu") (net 13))
 (segment (start 141.6565 94.293) (end 141.6565 95.1745) (width 0.5) (layer "F.Cu") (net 13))
 (segment (start 141.644 94.3055) (end 141.6565 94.293) (width 0.5) (layer "F.Cu") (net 13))
 (segment (start 144.7505 97.2305) (end 146.8635 97.2305) (width 0.5) (layer "F.Cu") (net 13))
 (segment (start 141.6565 95.1745) (end 142.24 95.758) (width 0.5) (layer "F.Cu") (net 13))
 (segment (start 206.632 116.964) (end 206.632 114.808) (width 1) (layer "F.Cu") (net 2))
 (segment (start 206.54 117.056) (end 206.632 116.964) (width 1) (layer "F.Cu") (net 2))
 (segment (start 206.54 118.644) (end 206.54 117.056) (width 1) (layer "F.Cu") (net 2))
 (segment (start 191.756 108.886) (end 191.756 106.92) (width 1) (layer "B.Cu") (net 2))
 (segment (start 191.756 108.886) (end 191.756 116.572) (width 1) (layer "B.Cu") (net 2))
 (segment (start 191.756 116.572) (end 192.692 117.508) (width 1) (layer "B.Cu") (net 2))
 (segment (start 191.756 106.92) (end 190.5 105.664) (width 1) (layer "B.Cu") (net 2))
 (segment (start 192.692 117.508) (end 192.692 122.4865) (width 1) (layer "B.Cu") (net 2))
 (segment (start 186.676 106.948) (end 186.676 108.886) (width 1) (layer "B.Cu") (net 2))
 (segment (start 187.96 105.664) (end 186.676 106.948) (width 1) (layer "B.Cu") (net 2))
 (segment (start 190.5 105.664) (end 187.96 105.664) (width 1) (layer "B.Cu") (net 2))
 (segment (start 131.9135 87.2885) (end 133.8395 87.2885) (width 0.5) (layer "F.Cu") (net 7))
 (segment (start 140.97 116.586) (end 136.906 112.522) (width 0.5) (layer "F.Cu") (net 7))
 (segment (start 130.048 89.154) (end 131.9135 87.2885) (width 0.5) (layer "F.Cu") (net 7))
 (segment (start 138.01 87.2885) (end 138.7625 88.041) (width 0.5) (layer "F.Cu") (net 7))
 (segment (start 151.384 115.316) (end 150.114 116.586) (width 0.5) (layer "F.Cu") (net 7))
 (segment (start 138.7625 88.041) (end 138.7625 88.8385) (width 0.5) (layer "F.Cu") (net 7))
 (segment (start 130.048 107.95) (end 130.048 89.154) (width 0.5) (layer "F.Cu") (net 7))
 (segment (start 147.87 111.944) (end 150.044 111.944) (width 0.5) (layer "F.Cu") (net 7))
 (segment (start 150.044 111.944) (end 151.384 113.284) (width 0.5) (layer "F.Cu") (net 7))
 (segment (start 150.114 116.586) (end 140.97 116.586) (width 0.5) (layer "F.Cu") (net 7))
 (segment (start 138.7625 88.8385) (end 141.8105 88.8385) (width 0.5) (layer "F.Cu") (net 7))
 (segment (start 136.906 112.522) (end 134.62 112.522) (width 0.5) (layer "F.Cu") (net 7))
 (segment (start 134.62 112.522) (end 130.048 107.95) (width 0.5) (layer "F.Cu") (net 7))
 (segment (start 151.384 113.284) (end 151.384 115.316) (width 0.5) (layer "F.Cu") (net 7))
 (segment (start 133.8395 87.2885) (end 138.01 87.2885) (width 0.5) (layer "F.Cu") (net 7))
 (segment (start 150.7225 88.2385) (end 151.3225 88.8385) (width 0.5) (layer "F.Cu") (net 14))
 (segment (start 151.3225 88.8385) (end 152.4785 88.8385) (width 0.5) (layer "F.Cu") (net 14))
 (segment (start 149.4305 88.2385) (end 150.7225 88.2385) (width 0.5) (layer "F.Cu") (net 14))
 (segment (start 149.552 96.6305) (end 150.7325 96.6305) (width 0.5) (layer "F.Cu") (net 14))
 (segment (start 150.7325 96.6305) (end 151.3325 97.2305) (width 0.5) (layer "F.Cu") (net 14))
 (segment (start 151.3325 97.2305) (end 152.4785 97.2305) (width 0.5) (layer "F.Cu") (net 14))
 (segment (start 138.5625 96.1445) (end 138.5625 97.2305) (width 0.5) (layer "F.Cu") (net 5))
 (segment (start 144.06 114.484) (end 140.519 114.484) (width 0.5) (layer "F.Cu") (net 5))
 (segment (start 134.874 111.252) (end 131.064 107.442) (width 0.5) (layer "F.Cu") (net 5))
 (segment (start 133.761 95.6805) (end 138.0985 95.6805) (width 0.5) (layer "F.Cu") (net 5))
 (segment (start 131.064 107.442) (end 131.064 96.52) (width 0.5) (layer "F.Cu") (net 5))
 (segment (start 138.0985 95.6805) (end 138.5625 96.1445) (width 0.5) (layer "F.Cu") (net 5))
 (segment (start 137.287 111.252) (end 134.874 111.252) (width 0.5) (layer "F.Cu") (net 5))
 (segment (start 131.064 96.52) (end 131.9035 95.6805) (width 0.5) (layer "F.Cu") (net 5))
 (segment (start 140.519 114.484) (end 137.287 111.252) (width 0.5) (layer "F.Cu") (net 5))
 (segment (start 131.9035 95.6805) (end 133.761 95.6805) (width 0.5) (layer "F.Cu") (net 5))
 (segment (start 208.44 123.644) (end 208.49 123.694) (width 2) (layer "F.Cu") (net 3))
 (segment (start 142.24 87.376) (end 144.526 87.376) (width 0.5) (layer "F.Cu") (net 11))
 (segment (start 144.8585 87.7085) (end 144.8585 88.8385) (width 0.5) (layer "F.Cu") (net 11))
 (segment (start 147.5555 88.1565) (end 146.8735 88.8385) (width 0.5) (layer "F.Cu") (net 11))
 (segment (start 141.8105 85.9135) (end 141.8105 86.9465) (width 0.5) (layer "F.Cu") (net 11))
 (segment (start 146.8735 88.8385) (end 144.8585 88.8385) (width 0.5) (layer "F.Cu") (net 11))
 (segment (start 144.526 87.376) (end 144.8585 87.7085) (width 0.5) (layer "F.Cu") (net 11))
 (segment (start 147.5555 87.2885) (end 147.5555 88.1565) (width 0.5) (layer "F.Cu") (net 11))
 (segment (start 141.8105 86.9465) (end 142.24 87.376) (width 0.5) (layer "F.Cu") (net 11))
 (segment (start 149.4305 86.3385) (end 150.6435 86.3385) (width 0.5) (layer "F.Cu") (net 15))
 (segment (start 150.6435 86.3385) (end 151.0685 85.9135) (width 0.5) (layer "F.Cu") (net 15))
 (segment (start 151.0685 85.9135) (end 152.4785 85.9135) (width 0.5) (layer "F.Cu") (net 15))
 (segment (start 150.3795 94.7305) (end 150.8045 94.3055) (width 0.5) (layer "F.Cu") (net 32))
 (segment (start 149.552 94.7305) (end 150.3795 94.7305) (width 0.5) (layer "F.Cu") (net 32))
 (segment (start 150.8045 94.3055) (end 152.4785 94.3055) (width 0.5) (layer "F.Cu") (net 32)))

